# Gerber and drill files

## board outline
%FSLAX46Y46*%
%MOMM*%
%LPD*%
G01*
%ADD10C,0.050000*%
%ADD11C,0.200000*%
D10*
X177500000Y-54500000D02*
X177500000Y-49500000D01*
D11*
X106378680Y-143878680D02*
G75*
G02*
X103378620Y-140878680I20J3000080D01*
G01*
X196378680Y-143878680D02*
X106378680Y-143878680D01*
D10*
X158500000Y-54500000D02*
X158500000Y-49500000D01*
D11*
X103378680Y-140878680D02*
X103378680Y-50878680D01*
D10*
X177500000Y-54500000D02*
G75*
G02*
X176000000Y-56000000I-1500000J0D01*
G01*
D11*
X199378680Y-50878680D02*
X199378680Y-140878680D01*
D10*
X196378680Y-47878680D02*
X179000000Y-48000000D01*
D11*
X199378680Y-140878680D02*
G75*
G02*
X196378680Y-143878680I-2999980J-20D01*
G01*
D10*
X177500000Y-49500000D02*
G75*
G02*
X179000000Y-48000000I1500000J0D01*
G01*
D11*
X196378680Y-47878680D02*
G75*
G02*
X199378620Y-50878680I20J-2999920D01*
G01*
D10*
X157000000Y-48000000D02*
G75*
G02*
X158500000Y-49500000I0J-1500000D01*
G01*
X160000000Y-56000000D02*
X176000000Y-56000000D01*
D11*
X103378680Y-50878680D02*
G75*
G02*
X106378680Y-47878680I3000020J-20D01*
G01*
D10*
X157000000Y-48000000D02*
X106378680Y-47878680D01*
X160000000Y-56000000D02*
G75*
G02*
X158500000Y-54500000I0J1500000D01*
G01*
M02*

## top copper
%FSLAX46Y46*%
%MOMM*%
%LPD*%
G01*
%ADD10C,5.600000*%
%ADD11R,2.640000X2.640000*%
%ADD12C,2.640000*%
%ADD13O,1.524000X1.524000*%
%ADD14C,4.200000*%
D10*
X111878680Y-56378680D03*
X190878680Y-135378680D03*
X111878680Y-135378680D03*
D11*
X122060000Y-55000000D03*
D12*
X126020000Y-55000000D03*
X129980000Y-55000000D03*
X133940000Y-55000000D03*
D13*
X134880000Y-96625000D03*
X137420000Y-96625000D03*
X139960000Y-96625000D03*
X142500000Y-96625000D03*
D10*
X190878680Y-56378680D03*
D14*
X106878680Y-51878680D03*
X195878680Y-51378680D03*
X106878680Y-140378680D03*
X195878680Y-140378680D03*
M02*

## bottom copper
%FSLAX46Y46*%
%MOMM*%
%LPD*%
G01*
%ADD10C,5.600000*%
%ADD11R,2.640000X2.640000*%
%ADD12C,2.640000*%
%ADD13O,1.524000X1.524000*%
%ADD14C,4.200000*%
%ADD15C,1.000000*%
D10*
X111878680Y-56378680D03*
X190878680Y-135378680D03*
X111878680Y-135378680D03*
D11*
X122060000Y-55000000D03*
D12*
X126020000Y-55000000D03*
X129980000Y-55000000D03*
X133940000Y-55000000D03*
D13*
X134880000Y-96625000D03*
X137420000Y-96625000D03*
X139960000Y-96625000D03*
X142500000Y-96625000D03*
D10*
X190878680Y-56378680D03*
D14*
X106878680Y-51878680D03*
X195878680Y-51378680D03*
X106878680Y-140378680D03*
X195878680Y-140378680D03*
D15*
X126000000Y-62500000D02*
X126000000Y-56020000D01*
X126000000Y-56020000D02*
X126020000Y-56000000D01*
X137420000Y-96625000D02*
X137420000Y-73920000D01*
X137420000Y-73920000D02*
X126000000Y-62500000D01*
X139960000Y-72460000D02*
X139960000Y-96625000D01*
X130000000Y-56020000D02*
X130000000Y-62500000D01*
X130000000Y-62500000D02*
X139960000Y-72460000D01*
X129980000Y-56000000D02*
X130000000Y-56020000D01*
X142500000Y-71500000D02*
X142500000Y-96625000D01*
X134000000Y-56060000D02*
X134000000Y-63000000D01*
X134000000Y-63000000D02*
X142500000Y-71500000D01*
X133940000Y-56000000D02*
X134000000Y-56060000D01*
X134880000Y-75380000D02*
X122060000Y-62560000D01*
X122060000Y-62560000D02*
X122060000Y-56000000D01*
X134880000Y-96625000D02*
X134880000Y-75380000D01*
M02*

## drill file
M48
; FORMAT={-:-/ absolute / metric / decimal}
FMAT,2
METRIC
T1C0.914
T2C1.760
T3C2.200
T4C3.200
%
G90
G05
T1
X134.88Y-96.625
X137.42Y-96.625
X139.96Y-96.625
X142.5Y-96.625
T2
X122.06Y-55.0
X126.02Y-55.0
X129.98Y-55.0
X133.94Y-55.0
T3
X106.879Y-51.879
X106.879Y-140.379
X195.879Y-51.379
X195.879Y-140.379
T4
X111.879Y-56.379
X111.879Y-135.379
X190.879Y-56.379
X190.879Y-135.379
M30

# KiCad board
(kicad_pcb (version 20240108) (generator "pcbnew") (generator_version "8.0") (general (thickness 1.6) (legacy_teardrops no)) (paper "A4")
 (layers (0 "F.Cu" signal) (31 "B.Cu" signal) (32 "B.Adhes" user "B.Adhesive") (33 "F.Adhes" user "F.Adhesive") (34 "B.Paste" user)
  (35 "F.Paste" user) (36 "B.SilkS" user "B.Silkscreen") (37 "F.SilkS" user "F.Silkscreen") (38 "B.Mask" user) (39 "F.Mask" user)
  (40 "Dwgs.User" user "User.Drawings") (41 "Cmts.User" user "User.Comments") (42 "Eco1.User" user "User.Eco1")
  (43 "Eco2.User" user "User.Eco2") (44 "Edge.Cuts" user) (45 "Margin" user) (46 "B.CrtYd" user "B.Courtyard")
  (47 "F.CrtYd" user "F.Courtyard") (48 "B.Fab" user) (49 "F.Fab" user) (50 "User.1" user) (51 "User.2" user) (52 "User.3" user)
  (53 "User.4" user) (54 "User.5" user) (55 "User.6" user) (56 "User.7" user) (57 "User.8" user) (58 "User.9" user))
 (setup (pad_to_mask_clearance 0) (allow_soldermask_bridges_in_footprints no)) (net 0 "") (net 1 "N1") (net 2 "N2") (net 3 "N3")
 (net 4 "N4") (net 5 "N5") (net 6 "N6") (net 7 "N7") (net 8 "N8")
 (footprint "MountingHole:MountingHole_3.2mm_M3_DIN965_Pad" (layer "F.Cu") (at 111.87868 56.37868)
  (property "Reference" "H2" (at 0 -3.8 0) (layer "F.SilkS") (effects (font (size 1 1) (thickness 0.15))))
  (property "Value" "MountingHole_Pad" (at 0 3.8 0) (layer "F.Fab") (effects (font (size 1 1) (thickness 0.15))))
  (pad "1" thru_hole circle (at 0 0) (size 5.6 5.6) (drill 3.2) (layers "*.Cu" "*.Mask") (remove_unused_layers no) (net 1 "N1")))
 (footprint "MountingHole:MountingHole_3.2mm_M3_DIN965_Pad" (layer "F.Cu") (at 190.87868 135.37868)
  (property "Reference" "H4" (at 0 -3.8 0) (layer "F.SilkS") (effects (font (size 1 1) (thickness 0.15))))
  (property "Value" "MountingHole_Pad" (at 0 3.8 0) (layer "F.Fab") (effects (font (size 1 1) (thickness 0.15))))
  (pad "1" thru_hole circle (at 0 0) (size 5.6 5.6) (drill 3.2) (layers "*.Cu" "*.Mask") (remove_unused_layers no) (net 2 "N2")))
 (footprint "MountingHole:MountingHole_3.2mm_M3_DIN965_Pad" (layer "F.Cu") (at 111.87868 135.37868)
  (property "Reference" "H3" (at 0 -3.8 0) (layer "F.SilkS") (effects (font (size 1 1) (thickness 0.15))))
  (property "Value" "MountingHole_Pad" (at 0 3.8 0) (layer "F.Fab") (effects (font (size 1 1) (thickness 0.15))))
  (pad "1" thru_hole circle (at 0 0) (size 5.6 5.6) (drill 3.2) (layers "*.Cu" "*.Mask") (remove_unused_layers no) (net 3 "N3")))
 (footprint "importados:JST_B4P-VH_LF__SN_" (layer "F.Cu") (at 128 55)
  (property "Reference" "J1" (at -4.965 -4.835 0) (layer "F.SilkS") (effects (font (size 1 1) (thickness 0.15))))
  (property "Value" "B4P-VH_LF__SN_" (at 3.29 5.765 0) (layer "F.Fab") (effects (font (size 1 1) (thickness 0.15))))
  (pad "1" thru_hole rect (at -5.94 0) (size 2.64 2.64) (drill 1.76) (layers "*.Cu" "*.Mask") (remove_unused_layers no) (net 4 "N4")
   (solder_mask_margin 0.102))
  (pad "2" thru_hole circle (at -1.98 0) (size 2.64 2.64) (drill 1.76) (layers "*.Cu" "*.Mask") (remove_unused_layers no) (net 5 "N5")
   (solder_mask_margin 0.102))
  (pad "3" thru_hole circle (at 1.98 0) (size 2.64 2.64) (drill 1.76) (layers "*.Cu" "*.Mask") (remove_unused_layers no) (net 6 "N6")
   (solder_mask_margin 0.102))
  (pad "4" thru_hole circle (at 5.94 0) (size 2.64 2.64) (drill 1.76) (layers "*.Cu" "*.Mask") (remove_unused_layers no) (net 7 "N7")
   (solder_mask_margin 0.102)))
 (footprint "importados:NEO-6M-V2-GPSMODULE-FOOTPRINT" (layer "F.Cu") (at 138.69 112.5)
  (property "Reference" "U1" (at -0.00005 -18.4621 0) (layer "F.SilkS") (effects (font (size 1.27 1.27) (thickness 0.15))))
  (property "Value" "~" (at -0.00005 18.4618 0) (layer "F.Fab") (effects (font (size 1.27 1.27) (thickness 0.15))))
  (pad "1" thru_hole oval (at -3.81 -15.875) (size 1.524 1.524) (drill 0.9144) (layers "*.Cu" "*.Mask") (remove_unused_layers no)
   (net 4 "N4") (solder_mask_margin 0.254) (thermal_bridge_angle 0))
  (pad "2" thru_hole oval (at -1.27 -15.875) (size 1.524 1.524) (drill 0.9144) (layers "*.Cu" "*.Mask") (remove_unused_layers no)
   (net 5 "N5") (solder_mask_margin 0.254) (thermal_bridge_angle 0))
  (pad "3" thru_hole oval (at 1.27 -15.875) (size 1.524 1.524) (drill 0.9144) (layers "*.Cu" "*.Mask") (remove_unused_layers no)
   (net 6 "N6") (solder_mask_margin 0.254) (thermal_bridge_angle 0))
  (pad "4" thru_hole oval (at 3.81 -15.875) (size 1.524 1.524) (drill 0.9144) (layers "*.Cu" "*.Mask") (remove_unused_layers no)
   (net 7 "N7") (solder_mask_margin 0.254) (thermal_bridge_angle 0))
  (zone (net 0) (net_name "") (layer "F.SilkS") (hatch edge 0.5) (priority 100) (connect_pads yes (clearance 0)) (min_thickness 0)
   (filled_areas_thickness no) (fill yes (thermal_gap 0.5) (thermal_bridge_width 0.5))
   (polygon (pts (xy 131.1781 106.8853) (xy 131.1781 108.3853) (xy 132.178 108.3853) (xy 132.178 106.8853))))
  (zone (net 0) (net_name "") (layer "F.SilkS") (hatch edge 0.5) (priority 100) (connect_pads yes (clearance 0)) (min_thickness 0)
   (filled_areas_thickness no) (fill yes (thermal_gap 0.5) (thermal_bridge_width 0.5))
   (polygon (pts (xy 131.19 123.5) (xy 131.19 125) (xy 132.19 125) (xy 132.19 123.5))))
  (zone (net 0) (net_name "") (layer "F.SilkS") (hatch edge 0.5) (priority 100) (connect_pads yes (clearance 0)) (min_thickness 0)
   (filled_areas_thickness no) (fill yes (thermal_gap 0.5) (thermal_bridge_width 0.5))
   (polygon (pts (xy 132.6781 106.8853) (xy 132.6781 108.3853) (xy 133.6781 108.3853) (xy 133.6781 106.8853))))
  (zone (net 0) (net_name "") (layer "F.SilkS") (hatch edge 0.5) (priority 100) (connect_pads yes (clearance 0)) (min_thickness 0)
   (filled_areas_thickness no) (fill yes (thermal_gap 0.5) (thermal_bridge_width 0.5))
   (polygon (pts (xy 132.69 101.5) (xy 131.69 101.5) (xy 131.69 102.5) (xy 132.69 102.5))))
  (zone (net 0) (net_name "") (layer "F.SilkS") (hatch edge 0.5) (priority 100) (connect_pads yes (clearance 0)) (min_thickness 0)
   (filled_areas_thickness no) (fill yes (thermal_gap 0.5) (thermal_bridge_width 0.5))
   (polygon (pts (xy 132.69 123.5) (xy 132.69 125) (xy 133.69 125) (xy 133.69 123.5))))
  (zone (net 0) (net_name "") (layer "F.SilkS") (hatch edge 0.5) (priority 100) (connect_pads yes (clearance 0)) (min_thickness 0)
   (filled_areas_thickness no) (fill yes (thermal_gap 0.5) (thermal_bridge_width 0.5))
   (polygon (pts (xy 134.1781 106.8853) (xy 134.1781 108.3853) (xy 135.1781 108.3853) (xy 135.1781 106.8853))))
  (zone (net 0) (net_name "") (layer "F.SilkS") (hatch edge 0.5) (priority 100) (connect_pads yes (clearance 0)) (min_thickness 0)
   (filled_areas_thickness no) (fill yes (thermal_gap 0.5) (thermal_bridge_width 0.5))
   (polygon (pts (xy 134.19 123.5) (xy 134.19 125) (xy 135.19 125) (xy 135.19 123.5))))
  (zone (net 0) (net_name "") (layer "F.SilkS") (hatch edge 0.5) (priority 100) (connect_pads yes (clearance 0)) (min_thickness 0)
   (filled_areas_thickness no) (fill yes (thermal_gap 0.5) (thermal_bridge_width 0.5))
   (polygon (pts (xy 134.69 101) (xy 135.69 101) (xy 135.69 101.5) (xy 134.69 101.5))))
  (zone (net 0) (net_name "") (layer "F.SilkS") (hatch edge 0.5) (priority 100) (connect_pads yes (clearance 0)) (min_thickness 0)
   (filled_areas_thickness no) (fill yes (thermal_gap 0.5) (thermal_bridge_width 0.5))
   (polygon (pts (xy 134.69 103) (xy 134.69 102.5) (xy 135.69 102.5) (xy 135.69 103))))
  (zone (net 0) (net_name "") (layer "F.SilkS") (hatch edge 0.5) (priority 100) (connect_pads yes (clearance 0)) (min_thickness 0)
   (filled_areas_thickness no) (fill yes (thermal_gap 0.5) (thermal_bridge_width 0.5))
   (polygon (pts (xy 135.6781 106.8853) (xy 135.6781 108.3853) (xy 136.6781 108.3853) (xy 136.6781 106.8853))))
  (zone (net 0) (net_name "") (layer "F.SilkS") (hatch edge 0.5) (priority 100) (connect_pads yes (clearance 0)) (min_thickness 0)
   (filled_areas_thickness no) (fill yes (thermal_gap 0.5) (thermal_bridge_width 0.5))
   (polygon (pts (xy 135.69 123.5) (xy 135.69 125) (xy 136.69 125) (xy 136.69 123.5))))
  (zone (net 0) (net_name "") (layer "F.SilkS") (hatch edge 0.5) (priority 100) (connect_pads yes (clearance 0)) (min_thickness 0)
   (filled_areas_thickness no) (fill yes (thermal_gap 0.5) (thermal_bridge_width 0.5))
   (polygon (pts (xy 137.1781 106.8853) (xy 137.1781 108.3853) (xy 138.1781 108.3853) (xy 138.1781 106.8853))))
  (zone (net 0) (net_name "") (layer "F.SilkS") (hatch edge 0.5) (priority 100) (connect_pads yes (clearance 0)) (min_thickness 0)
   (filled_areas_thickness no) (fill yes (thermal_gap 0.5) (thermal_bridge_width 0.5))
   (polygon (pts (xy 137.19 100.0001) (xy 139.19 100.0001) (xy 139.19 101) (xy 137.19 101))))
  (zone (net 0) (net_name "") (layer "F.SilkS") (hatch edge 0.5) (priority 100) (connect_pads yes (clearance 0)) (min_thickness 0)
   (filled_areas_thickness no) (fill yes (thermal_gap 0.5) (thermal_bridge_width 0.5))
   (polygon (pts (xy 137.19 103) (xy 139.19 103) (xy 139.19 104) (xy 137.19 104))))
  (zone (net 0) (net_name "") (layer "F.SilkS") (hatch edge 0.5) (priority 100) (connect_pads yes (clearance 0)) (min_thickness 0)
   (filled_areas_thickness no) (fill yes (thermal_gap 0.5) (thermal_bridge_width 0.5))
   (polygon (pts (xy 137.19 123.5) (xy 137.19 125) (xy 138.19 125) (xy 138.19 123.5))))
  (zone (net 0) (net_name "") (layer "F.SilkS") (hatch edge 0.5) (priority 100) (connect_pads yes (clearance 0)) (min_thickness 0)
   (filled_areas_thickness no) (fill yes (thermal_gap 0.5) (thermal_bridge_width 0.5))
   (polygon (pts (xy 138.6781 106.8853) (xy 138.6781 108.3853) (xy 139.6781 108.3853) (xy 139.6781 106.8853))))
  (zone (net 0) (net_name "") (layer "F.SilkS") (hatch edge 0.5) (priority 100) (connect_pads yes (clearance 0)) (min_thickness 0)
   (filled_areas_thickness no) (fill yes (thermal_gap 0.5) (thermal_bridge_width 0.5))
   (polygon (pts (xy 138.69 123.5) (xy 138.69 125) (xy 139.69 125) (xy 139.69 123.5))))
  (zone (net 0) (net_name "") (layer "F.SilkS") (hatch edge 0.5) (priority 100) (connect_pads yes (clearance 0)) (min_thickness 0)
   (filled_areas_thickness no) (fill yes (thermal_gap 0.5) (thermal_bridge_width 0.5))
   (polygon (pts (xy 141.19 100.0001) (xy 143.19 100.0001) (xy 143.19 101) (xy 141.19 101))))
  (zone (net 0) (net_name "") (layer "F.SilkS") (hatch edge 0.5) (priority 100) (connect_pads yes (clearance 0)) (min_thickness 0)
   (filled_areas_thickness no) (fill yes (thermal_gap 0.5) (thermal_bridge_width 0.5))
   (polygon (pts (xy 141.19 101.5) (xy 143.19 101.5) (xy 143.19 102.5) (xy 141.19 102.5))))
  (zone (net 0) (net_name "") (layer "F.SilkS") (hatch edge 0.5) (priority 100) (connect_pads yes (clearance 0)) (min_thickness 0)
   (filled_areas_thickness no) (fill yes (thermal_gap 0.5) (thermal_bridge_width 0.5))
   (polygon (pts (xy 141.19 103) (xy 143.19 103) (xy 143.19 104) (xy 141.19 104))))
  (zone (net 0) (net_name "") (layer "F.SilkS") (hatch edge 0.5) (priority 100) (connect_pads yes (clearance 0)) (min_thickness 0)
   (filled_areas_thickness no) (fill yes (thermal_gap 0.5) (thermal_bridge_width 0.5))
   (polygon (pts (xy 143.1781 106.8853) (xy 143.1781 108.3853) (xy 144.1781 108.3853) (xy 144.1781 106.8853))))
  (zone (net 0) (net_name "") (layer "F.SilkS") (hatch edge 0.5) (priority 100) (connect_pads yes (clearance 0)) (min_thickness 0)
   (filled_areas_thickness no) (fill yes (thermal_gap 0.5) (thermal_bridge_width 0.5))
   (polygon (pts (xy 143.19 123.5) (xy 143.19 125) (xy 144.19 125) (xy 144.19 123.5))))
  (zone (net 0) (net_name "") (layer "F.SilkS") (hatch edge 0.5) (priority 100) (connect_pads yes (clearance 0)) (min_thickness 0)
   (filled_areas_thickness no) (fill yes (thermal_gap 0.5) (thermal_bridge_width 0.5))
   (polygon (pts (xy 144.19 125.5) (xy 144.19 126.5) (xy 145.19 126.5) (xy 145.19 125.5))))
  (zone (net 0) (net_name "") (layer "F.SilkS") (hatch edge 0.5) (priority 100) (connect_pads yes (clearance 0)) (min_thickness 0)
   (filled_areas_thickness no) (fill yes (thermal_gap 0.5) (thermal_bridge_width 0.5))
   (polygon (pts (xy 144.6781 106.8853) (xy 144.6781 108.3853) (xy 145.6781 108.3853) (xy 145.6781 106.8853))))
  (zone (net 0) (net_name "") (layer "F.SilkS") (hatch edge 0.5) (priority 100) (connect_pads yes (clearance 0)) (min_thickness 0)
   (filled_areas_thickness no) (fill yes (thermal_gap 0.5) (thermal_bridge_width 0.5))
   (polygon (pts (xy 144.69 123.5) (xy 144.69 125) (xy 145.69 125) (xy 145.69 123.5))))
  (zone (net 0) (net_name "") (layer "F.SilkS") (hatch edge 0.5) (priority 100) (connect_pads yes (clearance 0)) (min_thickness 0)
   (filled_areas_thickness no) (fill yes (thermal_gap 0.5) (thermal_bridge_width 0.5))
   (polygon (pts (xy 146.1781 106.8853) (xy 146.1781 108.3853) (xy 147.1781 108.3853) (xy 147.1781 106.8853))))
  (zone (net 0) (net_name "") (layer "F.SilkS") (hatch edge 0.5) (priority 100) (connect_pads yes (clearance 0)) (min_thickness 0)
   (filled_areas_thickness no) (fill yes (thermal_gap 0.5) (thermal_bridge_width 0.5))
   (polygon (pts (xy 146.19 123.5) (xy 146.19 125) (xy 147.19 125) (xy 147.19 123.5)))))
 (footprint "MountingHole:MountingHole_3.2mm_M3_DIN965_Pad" (layer "F.Cu") (at 190.87868 56.37868)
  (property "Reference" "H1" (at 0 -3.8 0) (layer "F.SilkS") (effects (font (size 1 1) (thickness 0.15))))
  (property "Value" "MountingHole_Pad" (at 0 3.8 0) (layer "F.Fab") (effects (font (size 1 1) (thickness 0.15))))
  (pad "1" thru_hole circle (at 0 0) (size 5.6 5.6) (drill 3.2) (layers "*.Cu" "*.Mask") (remove_unused_layers no) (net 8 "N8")))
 (gr_line (start 177.5 54.5) (end 177.5 49.5) (stroke (width 0.05) (type default)) (layer "Edge.Cuts"))
 (gr_arc (start 106.37868 143.87868) (mid 104.257374 142.999986) (end 103.37868 140.87868) (stroke (width 0.2) (type default))
  (layer "Edge.Cuts"))
 (gr_line (start 196.37868 143.87868) (end 106.37868 143.87868) (stroke (width 0.2) (type default)) (layer "Edge.Cuts"))
 (gr_line (start 158.5 54.5) (end 158.5 49.5) (stroke (width 0.05) (type default)) (layer "Edge.Cuts"))
 (gr_line (start 103.37868 140.87868) (end 103.37868 50.87868) (stroke (width 0.2) (type default)) (layer "Edge.Cuts"))
 (gr_arc (start 177.5 54.5) (mid 177.06066 55.56066) (end 176 56) (stroke (width 0.05) (type default)) (layer "Edge.Cuts"))
 (gr_line (start 199.37868 50.87868) (end 199.37868 140.87868) (stroke (width 0.2) (type default)) (layer "Edge.Cuts"))
 (gr_line (start 196.37868 47.87868) (end 179 48) (stroke (width 0.05) (type default)) (layer "Edge.Cuts"))
 (gr_arc (start 199.37868 140.87868) (mid 198.500006 143.000006) (end 196.37868 143.87868) (stroke (width 0.2) (type default))
  (layer "Edge.Cuts"))
 (gr_arc (start 177.5 49.5) (mid 177.93934 48.43934) (end 179 48) (stroke (width 0.05) (type default)) (layer "Edge.Cuts"))
 (gr_arc (start 196.37868 47.87868) (mid 198.500014 48.757346) (end 199.37868 50.87868) (stroke (width 0.2) (type default))
  (layer "Edge.Cuts"))
 (gr_arc (start 157 48) (mid 158.06066 48.43934) (end 158.5 49.5) (stroke (width 0.05) (type default)) (layer "Edge.Cuts"))
 (gr_line (start 160 56) (end 176 56) (stroke (width 0.05) (type default)) (layer "Edge.Cuts"))
 (gr_arc (start 103.37868 50.87868) (mid 104.257366 48.757366) (end 106.37868 47.87868) (stroke (width 0.2) (type default))
  (layer "Edge.Cuts"))
 (gr_line (start 157 48) (end 106.37868 47.87868) (stroke (width 0.05) (type default)) (layer "Edge.Cuts"))
 (gr_arc (start 160 56) (mid 158.93934 55.56066) (end 158.5 54.5) (stroke (width 0.05) (type default)) (layer "Edge.Cuts"))
 (via (at 106.87868 51.87868) (size 4.2) (drill 2.2) (layers "F.Cu" "B.Cu") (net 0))
 (via (at 195.87868 51.37868) (size 4.2) (drill 2.2) (layers "F.Cu" "B.Cu") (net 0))
 (via (at 106.87868 140.37868) (size 4.2) (drill 2.2) (layers "F.Cu" "B.Cu") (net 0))
 (via (at 195.87868 140.37868) (size 4.2) (drill 2.2) (layers "F.Cu" "B.Cu") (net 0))
 (segment (start 126 62.5) (end 126 56.02) (width 1) (layer "B.Cu") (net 5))
 (segment (start 126 56.02) (end 126.02 56) (width 1) (layer "B.Cu") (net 5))
 (segment (start 137.42 96.625) (end 137.42 73.92) (width 1) (layer "B.Cu") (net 5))
 (segment (start 137.42 73.92) (end 126 62.5) (width 1) (layer "B.Cu") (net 5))
 (segment (start 139.96 72.46) (end 139.96 96.625) (width 1) (layer "B.Cu") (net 6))
 (segment (start 130 56.02) (end 130 62.5) (width 1) (layer "B.Cu") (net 6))
 (segment (start 130 62.5) (end 139.96 72.46) (width 1) (layer "B.Cu") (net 6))
 (segment (start 129.98 56) (end 130 56.02) (width 1) (layer "B.Cu") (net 6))
 (segment (start 142.5 71.5) (end 142.5 96.625) (width 1) (layer "B.Cu") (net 7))
 (segment (start 134 56.06) (end 134 63) (width 1) (layer "B.Cu") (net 7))
 (segment (start 134 63) (end 142.5 71.5) (width 1) (layer "B.Cu") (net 7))
 (segment (start 133.94 56) (end 134 56.06) (width 1) (layer "B.Cu") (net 7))
 (segment (start 134.88 75.38) (end 122.06 62.56) (width 1) (layer "B.Cu") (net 4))
 (segment (start 122.06 62.56) (end 122.06 56) (width 1) (layer "B.Cu") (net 4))
 (segment (start 134.88 96.625) (end 134.88 75.38) (width 1) (layer "B.Cu") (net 4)))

